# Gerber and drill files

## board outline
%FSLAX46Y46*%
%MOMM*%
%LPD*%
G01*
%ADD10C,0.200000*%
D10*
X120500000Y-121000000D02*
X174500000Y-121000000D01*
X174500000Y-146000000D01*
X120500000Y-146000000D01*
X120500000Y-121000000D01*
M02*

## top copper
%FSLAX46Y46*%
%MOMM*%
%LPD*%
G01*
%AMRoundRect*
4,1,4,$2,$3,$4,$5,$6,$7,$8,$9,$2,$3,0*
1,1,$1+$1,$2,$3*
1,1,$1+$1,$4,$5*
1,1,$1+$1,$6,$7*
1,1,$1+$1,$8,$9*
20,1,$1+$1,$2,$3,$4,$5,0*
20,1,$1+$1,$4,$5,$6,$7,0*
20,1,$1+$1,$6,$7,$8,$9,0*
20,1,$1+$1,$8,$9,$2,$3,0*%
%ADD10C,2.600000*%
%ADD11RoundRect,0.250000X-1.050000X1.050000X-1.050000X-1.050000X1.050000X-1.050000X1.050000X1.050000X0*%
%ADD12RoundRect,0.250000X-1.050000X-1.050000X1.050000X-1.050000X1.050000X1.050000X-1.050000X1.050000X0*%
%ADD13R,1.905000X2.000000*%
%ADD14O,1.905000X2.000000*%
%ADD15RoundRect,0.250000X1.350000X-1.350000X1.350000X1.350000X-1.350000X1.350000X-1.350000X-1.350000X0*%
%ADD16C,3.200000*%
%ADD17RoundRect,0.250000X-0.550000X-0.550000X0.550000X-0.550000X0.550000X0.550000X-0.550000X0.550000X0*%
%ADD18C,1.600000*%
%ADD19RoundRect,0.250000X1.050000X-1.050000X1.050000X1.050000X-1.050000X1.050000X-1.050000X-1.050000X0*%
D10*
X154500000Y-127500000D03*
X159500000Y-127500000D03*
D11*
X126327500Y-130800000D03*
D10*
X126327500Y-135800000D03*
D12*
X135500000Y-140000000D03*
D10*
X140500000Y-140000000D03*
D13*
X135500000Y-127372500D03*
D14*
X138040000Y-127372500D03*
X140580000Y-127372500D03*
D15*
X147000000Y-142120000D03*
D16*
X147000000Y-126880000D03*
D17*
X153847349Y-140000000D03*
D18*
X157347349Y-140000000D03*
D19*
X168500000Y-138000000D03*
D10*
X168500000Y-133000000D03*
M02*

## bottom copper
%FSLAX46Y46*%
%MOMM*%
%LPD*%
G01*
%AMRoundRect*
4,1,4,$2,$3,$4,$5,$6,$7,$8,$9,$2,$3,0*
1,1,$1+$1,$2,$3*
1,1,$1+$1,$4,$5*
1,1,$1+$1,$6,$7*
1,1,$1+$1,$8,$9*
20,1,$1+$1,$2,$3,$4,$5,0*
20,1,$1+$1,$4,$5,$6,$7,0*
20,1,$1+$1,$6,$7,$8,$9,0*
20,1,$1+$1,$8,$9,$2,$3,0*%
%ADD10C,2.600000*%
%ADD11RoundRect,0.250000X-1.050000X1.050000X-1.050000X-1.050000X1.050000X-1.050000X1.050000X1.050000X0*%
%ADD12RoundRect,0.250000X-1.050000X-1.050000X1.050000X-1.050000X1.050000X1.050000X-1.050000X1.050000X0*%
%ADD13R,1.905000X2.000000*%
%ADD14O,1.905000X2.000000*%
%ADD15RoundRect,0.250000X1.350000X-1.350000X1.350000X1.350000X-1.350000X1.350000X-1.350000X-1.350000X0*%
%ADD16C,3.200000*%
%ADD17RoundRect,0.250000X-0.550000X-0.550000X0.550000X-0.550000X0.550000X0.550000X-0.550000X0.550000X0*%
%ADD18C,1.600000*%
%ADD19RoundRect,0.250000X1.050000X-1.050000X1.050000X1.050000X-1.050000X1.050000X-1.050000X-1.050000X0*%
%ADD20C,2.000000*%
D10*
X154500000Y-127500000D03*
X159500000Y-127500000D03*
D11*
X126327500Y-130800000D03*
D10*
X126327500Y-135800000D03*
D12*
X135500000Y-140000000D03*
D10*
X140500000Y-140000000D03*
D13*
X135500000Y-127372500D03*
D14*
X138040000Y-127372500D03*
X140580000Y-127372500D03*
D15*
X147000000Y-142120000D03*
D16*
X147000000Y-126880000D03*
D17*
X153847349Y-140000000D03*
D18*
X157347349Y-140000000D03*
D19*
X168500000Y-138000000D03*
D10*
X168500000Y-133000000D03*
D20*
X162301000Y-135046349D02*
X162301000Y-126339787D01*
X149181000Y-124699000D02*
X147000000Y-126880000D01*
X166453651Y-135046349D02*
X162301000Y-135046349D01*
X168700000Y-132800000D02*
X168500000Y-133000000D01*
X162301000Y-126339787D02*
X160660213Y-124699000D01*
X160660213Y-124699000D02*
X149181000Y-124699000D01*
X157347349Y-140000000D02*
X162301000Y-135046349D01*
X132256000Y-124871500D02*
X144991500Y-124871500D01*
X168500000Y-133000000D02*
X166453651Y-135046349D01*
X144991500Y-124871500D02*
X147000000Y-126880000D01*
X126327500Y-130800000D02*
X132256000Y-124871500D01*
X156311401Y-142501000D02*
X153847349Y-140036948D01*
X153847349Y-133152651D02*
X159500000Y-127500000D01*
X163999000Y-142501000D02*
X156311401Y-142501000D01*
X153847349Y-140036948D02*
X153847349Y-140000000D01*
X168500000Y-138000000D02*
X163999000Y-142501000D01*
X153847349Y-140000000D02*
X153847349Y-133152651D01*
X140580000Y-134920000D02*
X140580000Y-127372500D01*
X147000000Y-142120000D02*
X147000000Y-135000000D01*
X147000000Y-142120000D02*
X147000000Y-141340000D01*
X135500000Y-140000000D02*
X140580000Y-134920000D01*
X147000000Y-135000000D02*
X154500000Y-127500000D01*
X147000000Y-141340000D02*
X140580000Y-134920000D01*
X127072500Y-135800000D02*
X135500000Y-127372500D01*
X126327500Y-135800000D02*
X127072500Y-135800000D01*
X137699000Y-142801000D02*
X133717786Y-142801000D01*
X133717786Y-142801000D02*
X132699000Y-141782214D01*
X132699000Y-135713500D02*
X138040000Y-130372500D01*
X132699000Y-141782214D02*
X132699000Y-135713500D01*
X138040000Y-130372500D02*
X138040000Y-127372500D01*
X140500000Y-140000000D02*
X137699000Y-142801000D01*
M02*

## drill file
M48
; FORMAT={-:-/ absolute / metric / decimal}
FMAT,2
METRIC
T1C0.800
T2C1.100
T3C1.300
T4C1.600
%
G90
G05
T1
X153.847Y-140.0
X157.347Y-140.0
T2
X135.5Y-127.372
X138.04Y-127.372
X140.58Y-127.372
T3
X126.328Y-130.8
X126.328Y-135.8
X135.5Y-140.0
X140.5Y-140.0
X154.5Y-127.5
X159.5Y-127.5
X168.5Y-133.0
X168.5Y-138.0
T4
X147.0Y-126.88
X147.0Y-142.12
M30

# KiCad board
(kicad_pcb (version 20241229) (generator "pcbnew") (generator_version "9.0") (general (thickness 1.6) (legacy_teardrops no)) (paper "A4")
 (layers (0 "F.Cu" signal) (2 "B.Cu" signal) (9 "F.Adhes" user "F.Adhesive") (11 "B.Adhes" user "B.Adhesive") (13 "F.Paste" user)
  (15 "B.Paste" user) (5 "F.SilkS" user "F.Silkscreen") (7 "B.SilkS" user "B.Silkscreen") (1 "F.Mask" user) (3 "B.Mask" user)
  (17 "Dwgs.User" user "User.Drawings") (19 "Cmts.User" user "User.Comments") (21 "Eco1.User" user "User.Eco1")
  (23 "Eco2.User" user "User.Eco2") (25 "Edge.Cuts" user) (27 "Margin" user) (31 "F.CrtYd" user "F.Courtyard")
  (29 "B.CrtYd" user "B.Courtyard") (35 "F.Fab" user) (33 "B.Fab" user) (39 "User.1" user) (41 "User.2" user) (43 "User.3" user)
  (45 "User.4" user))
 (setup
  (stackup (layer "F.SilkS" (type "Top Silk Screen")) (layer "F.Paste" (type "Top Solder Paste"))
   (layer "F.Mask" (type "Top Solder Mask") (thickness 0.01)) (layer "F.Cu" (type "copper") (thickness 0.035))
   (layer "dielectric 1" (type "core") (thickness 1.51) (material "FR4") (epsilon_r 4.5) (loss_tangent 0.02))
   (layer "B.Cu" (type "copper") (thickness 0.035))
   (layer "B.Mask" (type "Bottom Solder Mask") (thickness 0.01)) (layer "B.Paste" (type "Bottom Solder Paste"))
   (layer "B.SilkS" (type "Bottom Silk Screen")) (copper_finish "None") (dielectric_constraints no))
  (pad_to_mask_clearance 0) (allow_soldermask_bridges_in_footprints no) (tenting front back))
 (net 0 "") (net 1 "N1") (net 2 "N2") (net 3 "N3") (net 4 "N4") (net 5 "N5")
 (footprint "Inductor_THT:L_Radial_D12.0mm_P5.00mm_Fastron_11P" (layer "F.Cu") (at 154.5 127.5)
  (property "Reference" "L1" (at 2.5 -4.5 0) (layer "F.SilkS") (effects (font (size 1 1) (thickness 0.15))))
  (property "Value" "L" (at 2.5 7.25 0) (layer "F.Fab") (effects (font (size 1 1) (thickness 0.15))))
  (pad "1" thru_hole circle (at 0 0) (size 2.6 2.6) (drill 1.3) (layers "*.Cu" "*.Mask") (remove_unused_layers no) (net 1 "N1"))
  (pad "2" thru_hole circle (at 5 0) (size 2.6 2.6) (drill 1.3) (layers "*.Cu" "*.Mask") (remove_unused_layers no) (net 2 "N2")))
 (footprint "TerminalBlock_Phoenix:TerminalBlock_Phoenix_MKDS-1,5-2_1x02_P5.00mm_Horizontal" (layer "F.Cu") (at 126.3275 130.8 -90)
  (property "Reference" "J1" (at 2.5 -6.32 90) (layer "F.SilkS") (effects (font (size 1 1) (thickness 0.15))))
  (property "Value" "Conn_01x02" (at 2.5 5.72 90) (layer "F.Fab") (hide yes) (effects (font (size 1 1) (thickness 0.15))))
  (pad "1" thru_hole roundrect (at 0 0 270) (size 2.6 2.6) (drill 1.3) (layers "*.Cu" "*.Mask") (remove_unused_layers no)
   (roundrect_rratio 0.096154) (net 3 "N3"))
  (pad "2" thru_hole circle (at 5 0 270) (size 2.6 2.6) (drill 1.3) (layers "*.Cu" "*.Mask") (remove_unused_layers no) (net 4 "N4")))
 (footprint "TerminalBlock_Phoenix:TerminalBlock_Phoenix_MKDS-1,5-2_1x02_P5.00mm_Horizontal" (layer "F.Cu") (at 135.5 140)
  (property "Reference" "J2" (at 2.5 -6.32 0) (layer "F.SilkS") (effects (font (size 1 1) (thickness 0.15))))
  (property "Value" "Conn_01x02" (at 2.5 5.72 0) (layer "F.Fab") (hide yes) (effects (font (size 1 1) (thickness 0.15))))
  (pad "1" thru_hole roundrect (at 0 0) (size 2.6 2.6) (drill 1.3) (layers "*.Cu" "*.Mask") (remove_unused_layers no)
   (roundrect_rratio 0.096154) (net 1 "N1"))
  (pad "2" thru_hole circle (at 5 0) (size 2.6 2.6) (drill 1.3) (layers "*.Cu" "*.Mask") (remove_unused_layers no) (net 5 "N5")))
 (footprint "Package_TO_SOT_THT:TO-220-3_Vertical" (layer "F.Cu") (at 135.5 127.3725)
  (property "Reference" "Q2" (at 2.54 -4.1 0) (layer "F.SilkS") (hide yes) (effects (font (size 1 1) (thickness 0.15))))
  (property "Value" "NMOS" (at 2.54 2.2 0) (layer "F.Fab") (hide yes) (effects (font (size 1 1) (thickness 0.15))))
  (pad "1" thru_hole rect (at 0 0) (size 1.905 2) (drill 1.1) (layers "*.Cu" "*.Mask") (remove_unused_layers no) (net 4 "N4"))
  (pad "2" thru_hole oval (at 2.54 0) (size 1.905 2) (drill 1.1) (layers "*.Cu" "*.Mask") (remove_unused_layers no) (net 5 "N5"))
  (pad "3" thru_hole oval (at 5.08 0) (size 1.905 2) (drill 1.1) (layers "*.Cu" "*.Mask") (remove_unused_layers no) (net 1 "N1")))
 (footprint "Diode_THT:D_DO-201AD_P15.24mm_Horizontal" (layer "F.Cu") (at 147 142.12 90)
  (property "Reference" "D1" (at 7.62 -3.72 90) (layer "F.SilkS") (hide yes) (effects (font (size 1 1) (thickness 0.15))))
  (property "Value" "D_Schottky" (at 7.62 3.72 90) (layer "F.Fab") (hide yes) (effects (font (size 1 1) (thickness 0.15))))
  (pad "1" thru_hole roundrect (at 0 0 90) (size 3.2 3.2) (drill 1.6) (layers "*.Cu" "*.Mask") (remove_unused_layers no)
   (roundrect_rratio 0.078125) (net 1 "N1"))
  (pad "2" thru_hole circle (at 15.24 0 90) (size 3.2 3.2) (drill 1.6) (layers "*.Cu" "*.Mask") (remove_unused_layers no) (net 3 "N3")))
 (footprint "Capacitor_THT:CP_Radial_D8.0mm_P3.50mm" (layer "F.Cu") (at 153.847349 140)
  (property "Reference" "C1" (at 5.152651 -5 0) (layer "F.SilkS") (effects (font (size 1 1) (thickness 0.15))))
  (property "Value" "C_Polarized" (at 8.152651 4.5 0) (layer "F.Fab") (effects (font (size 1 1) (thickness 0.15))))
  (pad "1" thru_hole roundrect (at 0 0) (size 1.6 1.6) (drill 0.8) (layers "*.Cu" "*.Mask") (remove_unused_layers no)
   (roundrect_rratio 0.15625) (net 2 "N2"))
  (pad "2" thru_hole circle (at 3.5 0) (size 1.6 1.6) (drill 0.8) (layers "*.Cu" "*.Mask") (remove_unused_layers no) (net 3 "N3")))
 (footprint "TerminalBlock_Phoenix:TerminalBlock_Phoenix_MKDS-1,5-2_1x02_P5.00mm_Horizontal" (layer "F.Cu") (at 168.5 138 90)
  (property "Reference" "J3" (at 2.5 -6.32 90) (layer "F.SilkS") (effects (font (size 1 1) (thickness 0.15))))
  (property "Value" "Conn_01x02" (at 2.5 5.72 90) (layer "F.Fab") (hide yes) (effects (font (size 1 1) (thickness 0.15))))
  (pad "1" thru_hole roundrect (at 0 0 90) (size 2.6 2.6) (drill 1.3) (layers "*.Cu" "*.Mask") (remove_unused_layers no)
   (roundrect_rratio 0.096154) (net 2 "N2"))
  (pad "2" thru_hole circle (at 5 0 90) (size 2.6 2.6) (drill 1.3) (layers "*.Cu" "*.Mask") (remove_unused_layers no) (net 3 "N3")))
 (gr_rect (start 120.5 121) (end 174.5 146) (stroke (width 0.2) (type solid)) (fill no) (layer "Edge.Cuts"))
 (segment (start 162.301 135.046349) (end 162.301 126.339787) (width 2) (layer "B.Cu") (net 3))
 (segment (start 149.181 124.699) (end 147 126.88) (width 2) (layer "B.Cu") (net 3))
 (segment (start 166.453651 135.046349) (end 162.301 135.046349) (width 2) (layer "B.Cu") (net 3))
 (segment (start 168.7 132.8) (end 168.5 133) (width 2) (layer "B.Cu") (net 3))
 (segment (start 162.301 126.339787) (end 160.660213 124.699) (width 2) (layer "B.Cu") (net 3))
 (segment (start 160.660213 124.699) (end 149.181 124.699) (width 2) (layer "B.Cu") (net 3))
 (segment (start 157.347349 140) (end 162.301 135.046349) (width 2) (layer "B.Cu") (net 3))
 (segment (start 132.256 124.8715) (end 144.9915 124.8715) (width 2) (layer "B.Cu") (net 3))
 (segment (start 168.5 133) (end 166.453651 135.046349) (width 2) (layer "B.Cu") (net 3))
 (segment (start 144.9915 124.8715) (end 147 126.88) (width 2) (layer "B.Cu") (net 3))
 (segment (start 126.3275 130.8) (end 132.256 124.8715) (width 2) (layer "B.Cu") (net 3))
 (segment (start 156.311401 142.501) (end 153.847349 140.036948) (width 2) (layer "B.Cu") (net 2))
 (segment (start 153.847349 133.152651) (end 159.5 127.5) (width 2) (layer "B.Cu") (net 2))
 (segment (start 163.999 142.501) (end 156.311401 142.501) (width 2) (layer "B.Cu") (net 2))
 (segment (start 153.847349 140.036948) (end 153.847349 140) (width 2) (layer "B.Cu") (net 2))
 (segment (start 168.5 138) (end 163.999 142.501) (width 2) (layer "B.Cu") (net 2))
 (segment (start 153.847349 140) (end 153.847349 133.152651) (width 2) (layer "B.Cu") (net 2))
 (segment (start 140.58 134.92) (end 140.58 127.3725) (width 2) (layer "B.Cu") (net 1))
 (segment (start 147 142.12) (end 147 135) (width 2) (layer "B.Cu") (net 1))
 (segment (start 147 142.12) (end 147 141.34) (width 2) (layer "B.Cu") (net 1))
 (segment (start 135.5 140) (end 140.58 134.92) (width 2) (layer "B.Cu") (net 1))
 (segment (start 147 135) (end 154.5 127.5) (width 2) (layer "B.Cu") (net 1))
 (segment (start 147 141.34) (end 140.58 134.92) (width 2) (layer "B.Cu") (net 1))
 (segment (start 127.0725 135.8) (end 135.5 127.3725) (width 2) (layer "B.Cu") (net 4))
 (segment (start 126.3275 135.8) (end 127.0725 135.8) (width 2) (layer "B.Cu") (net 4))
 (segment (start 137.699 142.801) (end 133.717786 142.801) (width 2) (layer "B.Cu") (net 5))
 (segment (start 133.717786 142.801) (end 132.699 141.782214) (width 2) (layer "B.Cu") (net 5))
 (segment (start 132.699 135.7135) (end 138.04 130.3725) (width 2) (layer "B.Cu") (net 5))
 (segment (start 132.699 141.782214) (end 132.699 135.7135) (width 2) (layer "B.Cu") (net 5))
 (segment (start 138.04 130.3725) (end 138.04 127.3725) (width 2) (layer "B.Cu") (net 5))
 (segment (start 140.5 140) (end 137.699 142.801) (width 2) (layer "B.Cu") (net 5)))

